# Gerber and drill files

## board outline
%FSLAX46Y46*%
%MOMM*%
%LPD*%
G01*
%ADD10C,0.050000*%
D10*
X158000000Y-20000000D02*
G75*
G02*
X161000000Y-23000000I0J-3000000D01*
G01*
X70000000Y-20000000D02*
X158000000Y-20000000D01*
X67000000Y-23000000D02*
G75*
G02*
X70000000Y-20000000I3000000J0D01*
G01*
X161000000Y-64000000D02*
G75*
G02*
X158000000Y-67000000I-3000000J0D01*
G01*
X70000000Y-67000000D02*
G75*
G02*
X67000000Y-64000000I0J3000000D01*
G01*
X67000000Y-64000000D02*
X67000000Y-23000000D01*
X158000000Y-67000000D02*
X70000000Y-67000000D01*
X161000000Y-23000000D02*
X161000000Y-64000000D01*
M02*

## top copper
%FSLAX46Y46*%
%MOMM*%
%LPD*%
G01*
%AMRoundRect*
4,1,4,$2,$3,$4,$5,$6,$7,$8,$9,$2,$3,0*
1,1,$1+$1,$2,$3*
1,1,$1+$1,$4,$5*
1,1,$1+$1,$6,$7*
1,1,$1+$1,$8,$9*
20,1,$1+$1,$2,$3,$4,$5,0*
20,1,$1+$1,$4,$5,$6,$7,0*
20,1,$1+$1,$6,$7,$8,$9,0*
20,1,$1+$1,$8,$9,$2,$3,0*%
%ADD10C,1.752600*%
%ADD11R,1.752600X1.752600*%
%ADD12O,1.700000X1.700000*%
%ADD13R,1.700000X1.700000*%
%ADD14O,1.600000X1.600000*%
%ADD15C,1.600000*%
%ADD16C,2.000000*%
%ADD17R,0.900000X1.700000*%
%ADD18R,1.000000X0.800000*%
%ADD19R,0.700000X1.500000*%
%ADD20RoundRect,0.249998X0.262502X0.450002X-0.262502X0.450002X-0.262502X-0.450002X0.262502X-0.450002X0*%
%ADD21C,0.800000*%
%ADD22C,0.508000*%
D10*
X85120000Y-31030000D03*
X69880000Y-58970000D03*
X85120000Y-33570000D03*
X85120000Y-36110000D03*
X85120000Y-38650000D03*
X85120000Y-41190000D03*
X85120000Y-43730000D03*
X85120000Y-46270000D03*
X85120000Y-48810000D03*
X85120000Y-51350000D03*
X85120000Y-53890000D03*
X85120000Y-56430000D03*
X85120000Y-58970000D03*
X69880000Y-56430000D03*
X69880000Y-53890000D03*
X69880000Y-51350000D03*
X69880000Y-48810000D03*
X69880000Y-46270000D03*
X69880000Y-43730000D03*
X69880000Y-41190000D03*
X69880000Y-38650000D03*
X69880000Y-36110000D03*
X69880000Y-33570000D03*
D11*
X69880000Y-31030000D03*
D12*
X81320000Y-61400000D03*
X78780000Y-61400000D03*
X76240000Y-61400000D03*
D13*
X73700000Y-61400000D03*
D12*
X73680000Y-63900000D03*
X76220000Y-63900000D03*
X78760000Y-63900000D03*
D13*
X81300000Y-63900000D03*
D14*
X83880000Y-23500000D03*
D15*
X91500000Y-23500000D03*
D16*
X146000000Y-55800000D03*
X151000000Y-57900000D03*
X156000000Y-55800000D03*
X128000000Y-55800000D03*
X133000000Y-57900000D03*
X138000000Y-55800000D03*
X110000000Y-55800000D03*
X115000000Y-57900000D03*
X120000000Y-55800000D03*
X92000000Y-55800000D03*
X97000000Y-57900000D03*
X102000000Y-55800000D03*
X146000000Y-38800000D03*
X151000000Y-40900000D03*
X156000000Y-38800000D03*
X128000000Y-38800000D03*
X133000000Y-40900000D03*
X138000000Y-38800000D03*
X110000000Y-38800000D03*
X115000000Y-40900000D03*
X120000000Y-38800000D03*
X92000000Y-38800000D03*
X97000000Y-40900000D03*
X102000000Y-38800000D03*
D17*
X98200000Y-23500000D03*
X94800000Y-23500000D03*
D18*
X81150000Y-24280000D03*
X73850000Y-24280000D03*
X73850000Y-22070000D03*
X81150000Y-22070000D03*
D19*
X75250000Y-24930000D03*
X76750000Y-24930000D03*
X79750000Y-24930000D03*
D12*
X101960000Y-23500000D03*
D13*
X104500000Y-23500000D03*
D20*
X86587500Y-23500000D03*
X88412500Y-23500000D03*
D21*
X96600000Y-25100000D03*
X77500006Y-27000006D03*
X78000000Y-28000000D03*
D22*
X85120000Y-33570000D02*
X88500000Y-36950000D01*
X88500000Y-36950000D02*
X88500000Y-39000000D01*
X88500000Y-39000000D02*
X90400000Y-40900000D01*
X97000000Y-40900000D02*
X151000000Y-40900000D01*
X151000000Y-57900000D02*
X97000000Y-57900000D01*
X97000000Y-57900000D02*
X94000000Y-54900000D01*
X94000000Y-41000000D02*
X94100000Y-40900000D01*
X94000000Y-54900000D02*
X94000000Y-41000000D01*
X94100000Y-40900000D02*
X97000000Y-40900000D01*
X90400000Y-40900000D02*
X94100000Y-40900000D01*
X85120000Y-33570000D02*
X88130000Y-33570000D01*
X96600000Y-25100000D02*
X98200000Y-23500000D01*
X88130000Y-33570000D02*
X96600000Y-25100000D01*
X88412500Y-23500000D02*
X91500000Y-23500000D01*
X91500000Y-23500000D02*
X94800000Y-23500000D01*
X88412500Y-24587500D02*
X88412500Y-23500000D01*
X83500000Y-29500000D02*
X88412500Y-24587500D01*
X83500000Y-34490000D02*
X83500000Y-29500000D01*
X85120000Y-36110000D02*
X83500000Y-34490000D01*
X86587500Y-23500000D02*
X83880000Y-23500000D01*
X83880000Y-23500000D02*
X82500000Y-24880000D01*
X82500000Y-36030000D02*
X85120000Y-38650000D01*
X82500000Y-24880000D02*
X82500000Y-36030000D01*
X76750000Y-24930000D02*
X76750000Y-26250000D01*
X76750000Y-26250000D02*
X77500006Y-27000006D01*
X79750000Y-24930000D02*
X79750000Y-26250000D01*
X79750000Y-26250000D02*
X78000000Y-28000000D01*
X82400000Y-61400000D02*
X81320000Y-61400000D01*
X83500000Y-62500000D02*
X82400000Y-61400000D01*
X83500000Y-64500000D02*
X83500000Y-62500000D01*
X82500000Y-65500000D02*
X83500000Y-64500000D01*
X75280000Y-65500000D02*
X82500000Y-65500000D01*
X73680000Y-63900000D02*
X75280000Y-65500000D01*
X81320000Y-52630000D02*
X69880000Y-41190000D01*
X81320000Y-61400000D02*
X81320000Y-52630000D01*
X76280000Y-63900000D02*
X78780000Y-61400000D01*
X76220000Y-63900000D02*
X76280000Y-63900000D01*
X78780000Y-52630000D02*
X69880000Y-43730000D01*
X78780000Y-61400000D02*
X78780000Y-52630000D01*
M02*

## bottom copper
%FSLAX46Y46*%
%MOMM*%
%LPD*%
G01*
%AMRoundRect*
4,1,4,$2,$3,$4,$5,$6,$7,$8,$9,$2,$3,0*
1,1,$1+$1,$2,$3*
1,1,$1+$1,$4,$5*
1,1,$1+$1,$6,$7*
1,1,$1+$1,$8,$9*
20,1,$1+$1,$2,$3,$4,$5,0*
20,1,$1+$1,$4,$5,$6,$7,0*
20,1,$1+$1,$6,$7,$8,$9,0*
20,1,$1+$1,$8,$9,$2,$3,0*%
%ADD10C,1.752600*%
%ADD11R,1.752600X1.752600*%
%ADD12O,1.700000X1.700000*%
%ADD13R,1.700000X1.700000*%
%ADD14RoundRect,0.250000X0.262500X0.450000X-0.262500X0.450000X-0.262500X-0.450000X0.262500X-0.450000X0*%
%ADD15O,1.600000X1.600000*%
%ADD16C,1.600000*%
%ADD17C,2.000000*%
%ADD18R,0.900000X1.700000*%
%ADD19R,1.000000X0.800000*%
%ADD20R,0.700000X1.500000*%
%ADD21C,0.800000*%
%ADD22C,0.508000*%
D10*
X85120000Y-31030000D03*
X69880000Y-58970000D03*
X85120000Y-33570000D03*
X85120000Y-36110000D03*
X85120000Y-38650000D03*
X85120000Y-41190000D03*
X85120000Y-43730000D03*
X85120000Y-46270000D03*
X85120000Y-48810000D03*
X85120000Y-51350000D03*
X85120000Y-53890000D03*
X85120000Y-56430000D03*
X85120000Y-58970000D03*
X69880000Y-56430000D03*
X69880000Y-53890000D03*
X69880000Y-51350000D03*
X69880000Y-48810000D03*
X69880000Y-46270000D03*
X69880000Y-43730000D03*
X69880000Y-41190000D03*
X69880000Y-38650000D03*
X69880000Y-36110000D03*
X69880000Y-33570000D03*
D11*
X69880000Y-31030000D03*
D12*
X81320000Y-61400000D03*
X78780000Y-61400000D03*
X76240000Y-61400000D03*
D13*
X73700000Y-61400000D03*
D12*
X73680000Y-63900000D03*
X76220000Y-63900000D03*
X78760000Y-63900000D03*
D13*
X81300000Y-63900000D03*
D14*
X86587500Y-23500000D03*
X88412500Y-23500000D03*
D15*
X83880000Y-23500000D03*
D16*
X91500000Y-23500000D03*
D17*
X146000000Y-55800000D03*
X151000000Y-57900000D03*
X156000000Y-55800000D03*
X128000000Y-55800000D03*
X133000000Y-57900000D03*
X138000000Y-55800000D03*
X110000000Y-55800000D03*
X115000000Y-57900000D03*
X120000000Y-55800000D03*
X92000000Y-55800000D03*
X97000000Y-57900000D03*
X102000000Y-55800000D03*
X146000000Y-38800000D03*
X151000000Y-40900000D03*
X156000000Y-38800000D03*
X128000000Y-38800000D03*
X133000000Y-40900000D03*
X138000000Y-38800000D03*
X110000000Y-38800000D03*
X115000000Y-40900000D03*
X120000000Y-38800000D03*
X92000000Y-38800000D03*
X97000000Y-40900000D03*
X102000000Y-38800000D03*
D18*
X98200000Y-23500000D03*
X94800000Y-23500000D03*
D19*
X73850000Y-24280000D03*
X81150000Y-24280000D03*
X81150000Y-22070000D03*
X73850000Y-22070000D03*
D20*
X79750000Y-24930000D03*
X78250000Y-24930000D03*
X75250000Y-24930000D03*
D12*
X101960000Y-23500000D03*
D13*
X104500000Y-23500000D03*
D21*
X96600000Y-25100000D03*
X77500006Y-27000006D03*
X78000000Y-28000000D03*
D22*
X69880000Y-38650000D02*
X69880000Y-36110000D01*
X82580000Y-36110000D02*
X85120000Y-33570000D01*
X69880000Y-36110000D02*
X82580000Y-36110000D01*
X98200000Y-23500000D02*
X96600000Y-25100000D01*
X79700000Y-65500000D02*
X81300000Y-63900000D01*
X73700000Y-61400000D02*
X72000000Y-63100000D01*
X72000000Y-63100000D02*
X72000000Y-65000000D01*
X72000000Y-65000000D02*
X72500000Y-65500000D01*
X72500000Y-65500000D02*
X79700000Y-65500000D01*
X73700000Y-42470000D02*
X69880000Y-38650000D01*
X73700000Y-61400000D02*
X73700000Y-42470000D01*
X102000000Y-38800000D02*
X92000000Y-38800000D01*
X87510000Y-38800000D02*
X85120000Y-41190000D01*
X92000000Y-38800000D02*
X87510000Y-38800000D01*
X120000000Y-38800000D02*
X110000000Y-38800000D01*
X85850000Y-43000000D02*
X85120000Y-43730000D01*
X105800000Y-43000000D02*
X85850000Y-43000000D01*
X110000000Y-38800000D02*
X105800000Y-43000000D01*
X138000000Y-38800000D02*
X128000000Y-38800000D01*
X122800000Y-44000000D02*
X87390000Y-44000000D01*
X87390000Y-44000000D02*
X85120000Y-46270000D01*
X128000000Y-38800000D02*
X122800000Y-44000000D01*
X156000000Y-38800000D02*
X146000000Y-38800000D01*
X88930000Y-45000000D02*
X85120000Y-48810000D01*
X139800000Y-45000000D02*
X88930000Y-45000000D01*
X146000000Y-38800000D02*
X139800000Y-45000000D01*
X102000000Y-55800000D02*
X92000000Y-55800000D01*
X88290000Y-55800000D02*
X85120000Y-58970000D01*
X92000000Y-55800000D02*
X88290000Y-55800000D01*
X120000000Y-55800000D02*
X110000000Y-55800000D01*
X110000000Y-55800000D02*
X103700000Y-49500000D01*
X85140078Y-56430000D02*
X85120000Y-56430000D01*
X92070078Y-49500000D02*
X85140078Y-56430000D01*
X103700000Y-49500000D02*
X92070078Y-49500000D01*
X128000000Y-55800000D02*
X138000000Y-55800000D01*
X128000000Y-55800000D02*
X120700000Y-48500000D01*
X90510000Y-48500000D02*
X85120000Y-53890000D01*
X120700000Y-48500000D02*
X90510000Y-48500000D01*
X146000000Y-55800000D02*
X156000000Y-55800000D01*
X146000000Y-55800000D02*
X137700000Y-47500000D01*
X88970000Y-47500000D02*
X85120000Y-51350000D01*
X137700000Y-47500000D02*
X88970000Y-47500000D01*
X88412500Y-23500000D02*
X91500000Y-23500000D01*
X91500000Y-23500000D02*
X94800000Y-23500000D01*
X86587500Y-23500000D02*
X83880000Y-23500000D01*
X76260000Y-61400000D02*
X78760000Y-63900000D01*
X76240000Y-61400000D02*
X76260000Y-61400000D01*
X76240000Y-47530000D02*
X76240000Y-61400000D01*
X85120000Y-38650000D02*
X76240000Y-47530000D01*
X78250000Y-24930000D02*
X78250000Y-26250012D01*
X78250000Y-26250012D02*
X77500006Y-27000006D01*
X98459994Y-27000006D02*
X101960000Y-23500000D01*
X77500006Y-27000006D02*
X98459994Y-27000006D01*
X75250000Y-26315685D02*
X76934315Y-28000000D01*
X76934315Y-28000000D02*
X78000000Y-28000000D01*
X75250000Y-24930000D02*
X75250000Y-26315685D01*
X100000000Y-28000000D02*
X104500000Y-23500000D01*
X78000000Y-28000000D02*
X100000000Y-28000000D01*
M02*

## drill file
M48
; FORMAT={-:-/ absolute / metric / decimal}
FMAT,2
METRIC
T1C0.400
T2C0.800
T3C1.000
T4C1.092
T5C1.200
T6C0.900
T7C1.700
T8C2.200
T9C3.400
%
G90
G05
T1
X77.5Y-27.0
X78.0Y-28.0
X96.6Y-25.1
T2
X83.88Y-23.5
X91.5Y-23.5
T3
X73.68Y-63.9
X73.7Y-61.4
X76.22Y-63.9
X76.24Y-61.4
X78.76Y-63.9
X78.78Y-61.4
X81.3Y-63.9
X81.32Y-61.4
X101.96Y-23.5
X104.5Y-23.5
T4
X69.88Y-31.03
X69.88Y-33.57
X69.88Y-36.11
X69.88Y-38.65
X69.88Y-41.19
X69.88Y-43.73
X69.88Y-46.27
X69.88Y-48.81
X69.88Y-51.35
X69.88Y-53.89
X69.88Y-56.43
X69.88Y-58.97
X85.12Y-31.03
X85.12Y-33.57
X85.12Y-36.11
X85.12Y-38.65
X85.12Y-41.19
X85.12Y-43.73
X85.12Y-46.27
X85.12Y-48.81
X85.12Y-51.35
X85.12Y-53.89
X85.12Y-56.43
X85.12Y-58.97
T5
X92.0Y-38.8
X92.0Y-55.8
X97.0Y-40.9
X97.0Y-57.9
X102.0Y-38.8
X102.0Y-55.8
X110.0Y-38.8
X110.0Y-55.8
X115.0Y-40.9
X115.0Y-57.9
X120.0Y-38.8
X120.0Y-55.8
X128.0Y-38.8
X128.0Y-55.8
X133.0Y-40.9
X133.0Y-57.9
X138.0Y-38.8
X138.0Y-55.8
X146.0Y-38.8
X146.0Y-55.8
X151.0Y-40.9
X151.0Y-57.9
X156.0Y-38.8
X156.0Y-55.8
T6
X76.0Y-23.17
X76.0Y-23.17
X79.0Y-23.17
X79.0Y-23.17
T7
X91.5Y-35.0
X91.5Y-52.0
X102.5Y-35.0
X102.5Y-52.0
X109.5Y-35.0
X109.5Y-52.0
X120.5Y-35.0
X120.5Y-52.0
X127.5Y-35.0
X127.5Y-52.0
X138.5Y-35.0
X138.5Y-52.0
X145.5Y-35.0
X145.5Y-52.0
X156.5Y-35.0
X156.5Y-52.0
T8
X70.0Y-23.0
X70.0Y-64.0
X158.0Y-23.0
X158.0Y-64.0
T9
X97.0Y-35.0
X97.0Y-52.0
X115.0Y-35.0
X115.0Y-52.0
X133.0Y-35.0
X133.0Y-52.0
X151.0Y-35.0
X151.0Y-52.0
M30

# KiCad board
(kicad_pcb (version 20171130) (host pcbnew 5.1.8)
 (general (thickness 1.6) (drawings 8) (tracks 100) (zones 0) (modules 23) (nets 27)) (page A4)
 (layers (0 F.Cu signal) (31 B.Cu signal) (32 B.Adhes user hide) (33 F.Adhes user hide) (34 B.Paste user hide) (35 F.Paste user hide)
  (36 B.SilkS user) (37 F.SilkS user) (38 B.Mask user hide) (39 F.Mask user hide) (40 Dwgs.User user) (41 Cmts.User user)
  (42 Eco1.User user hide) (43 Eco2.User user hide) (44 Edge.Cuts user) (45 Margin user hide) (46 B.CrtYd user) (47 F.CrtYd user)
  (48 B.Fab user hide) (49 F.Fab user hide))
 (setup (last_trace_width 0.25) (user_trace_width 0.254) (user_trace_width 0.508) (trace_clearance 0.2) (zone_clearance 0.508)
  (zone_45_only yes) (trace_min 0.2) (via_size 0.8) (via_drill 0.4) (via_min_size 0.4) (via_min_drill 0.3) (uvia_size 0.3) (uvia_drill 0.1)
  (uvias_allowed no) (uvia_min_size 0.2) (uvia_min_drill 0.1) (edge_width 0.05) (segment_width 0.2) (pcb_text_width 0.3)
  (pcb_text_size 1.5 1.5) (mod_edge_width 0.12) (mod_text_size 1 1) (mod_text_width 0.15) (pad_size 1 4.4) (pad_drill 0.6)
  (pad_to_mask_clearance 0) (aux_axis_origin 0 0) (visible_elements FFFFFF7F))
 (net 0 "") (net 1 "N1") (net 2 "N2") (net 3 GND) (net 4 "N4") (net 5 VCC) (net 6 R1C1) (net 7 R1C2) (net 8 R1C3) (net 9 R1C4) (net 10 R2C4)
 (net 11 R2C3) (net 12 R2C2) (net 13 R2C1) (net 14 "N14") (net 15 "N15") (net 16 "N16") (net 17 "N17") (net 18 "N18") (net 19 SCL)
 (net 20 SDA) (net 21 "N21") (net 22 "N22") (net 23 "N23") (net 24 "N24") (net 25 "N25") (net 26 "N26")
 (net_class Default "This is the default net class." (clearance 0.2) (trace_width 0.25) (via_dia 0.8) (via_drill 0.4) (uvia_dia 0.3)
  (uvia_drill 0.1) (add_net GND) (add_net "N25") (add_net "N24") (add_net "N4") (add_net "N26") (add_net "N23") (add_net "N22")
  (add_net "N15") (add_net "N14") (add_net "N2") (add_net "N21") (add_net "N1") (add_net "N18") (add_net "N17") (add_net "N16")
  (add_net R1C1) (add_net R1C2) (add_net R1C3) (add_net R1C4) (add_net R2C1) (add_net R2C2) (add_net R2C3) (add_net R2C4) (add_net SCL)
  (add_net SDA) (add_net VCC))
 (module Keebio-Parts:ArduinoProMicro (layer F.Cu) (at 77.5 45 270)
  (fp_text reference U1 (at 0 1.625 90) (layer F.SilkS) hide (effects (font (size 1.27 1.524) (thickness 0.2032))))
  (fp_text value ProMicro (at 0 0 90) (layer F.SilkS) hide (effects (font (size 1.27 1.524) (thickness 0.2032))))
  (pad 24 thru_hole circle (at -13.97 -7.62 270) (size 1.7526 1.7526) (drill 1.0922) (layers *.Cu *.SilkS *.Mask) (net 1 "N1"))
  (pad 12 thru_hole circle (at 13.97 7.62 270) (size 1.7526 1.7526) (drill 1.0922) (layers *.Cu *.SilkS *.Mask) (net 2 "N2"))
  (pad 23 thru_hole circle (at -11.43 -7.62 270) (size 1.7526 1.7526) (drill 1.0922) (layers *.Cu *.SilkS *.Mask) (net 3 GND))
  (pad 22 thru_hole circle (at -8.89 -7.62 270) (size 1.7526 1.7526) (drill 1.0922) (layers *.Cu *.SilkS *.Mask) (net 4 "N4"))
  (pad 21 thru_hole circle (at -6.35 -7.62 270) (size 1.7526 1.7526) (drill 1.0922) (layers *.Cu *.SilkS *.Mask) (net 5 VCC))
  (pad 20 thru_hole circle (at -3.81 -7.62 270) (size 1.7526 1.7526) (drill 1.0922) (layers *.Cu *.SilkS *.Mask) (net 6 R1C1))
  (pad 19 thru_hole circle (at -1.27 -7.62 270) (size 1.7526 1.7526) (drill 1.0922) (layers *.Cu *.SilkS *.Mask) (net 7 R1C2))
  (pad 18 thru_hole circle (at 1.27 -7.62 270) (size 1.7526 1.7526) (drill 1.0922) (layers *.Cu *.SilkS *.Mask) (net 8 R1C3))
  (pad 17 thru_hole circle (at 3.81 -7.62 270) (size 1.7526 1.7526) (drill 1.0922) (layers *.Cu *.SilkS *.Mask) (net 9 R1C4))
  (pad 16 thru_hole circle (at 6.35 -7.62 270) (size 1.7526 1.7526) (drill 1.0922) (layers *.Cu *.SilkS *.Mask) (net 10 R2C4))
  (pad 15 thru_hole circle (at 8.89 -7.62 270) (size 1.7526 1.7526) (drill 1.0922) (layers *.Cu *.SilkS *.Mask) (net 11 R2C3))
  (pad 14 thru_hole circle (at 11.43 -7.62 270) (size 1.7526 1.7526) (drill 1.0922) (layers *.Cu *.SilkS *.Mask) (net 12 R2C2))
  (pad 13 thru_hole circle (at 13.97 -7.62 270) (size 1.7526 1.7526) (drill 1.0922) (layers *.Cu *.SilkS *.Mask) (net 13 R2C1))
  (pad 11 thru_hole circle (at 11.43 7.62 270) (size 1.7526 1.7526) (drill 1.0922) (layers *.Cu *.SilkS *.Mask) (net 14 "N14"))
  (pad 10 thru_hole circle (at 8.89 7.62 270) (size 1.7526 1.7526) (drill 1.0922) (layers *.Cu *.SilkS *.Mask) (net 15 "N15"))
  (pad 9 thru_hole circle (at 6.35 7.62 270) (size 1.7526 1.7526) (drill 1.0922) (layers *.Cu *.SilkS *.Mask) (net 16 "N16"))
  (pad 8 thru_hole circle (at 3.81 7.62 270) (size 1.7526 1.7526) (drill 1.0922) (layers *.Cu *.SilkS *.Mask) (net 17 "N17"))
  (pad 7 thru_hole circle (at 1.27 7.62 270) (size 1.7526 1.7526) (drill 1.0922) (layers *.Cu *.SilkS *.Mask) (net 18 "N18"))
  (pad 6 thru_hole circle (at -1.27 7.62 270) (size 1.7526 1.7526) (drill 1.0922) (layers *.Cu *.SilkS *.Mask) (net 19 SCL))
  (pad 5 thru_hole circle (at -3.81 7.62 270) (size 1.7526 1.7526) (drill 1.0922) (layers *.Cu *.SilkS *.Mask) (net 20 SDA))
  (pad 4 thru_hole circle (at -6.35 7.62 270) (size 1.7526 1.7526) (drill 1.0922) (layers *.Cu *.SilkS *.Mask) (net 3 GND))
  (pad 3 thru_hole circle (at -8.89 7.62 270) (size 1.7526 1.7526) (drill 1.0922) (layers *.Cu *.SilkS *.Mask) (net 3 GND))
  (pad 2 thru_hole circle (at -11.43 7.62 270) (size 1.7526 1.7526) (drill 1.0922) (layers *.Cu *.SilkS *.Mask) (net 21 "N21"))
  (pad 1 thru_hole rect (at -13.97 7.62 270) (size 1.7526 1.7526) (drill 1.0922) (layers *.Cu *.SilkS *.Mask) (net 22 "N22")))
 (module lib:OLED (layer B.Cu) (at 83.5 63 90)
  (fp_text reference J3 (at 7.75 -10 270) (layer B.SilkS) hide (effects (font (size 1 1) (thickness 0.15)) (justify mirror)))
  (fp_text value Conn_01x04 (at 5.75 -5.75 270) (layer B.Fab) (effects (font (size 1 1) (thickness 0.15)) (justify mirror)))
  (pad 4 thru_hole oval (at 1.6 -2.18 270) (size 1.7 1.7) (drill 1) (layers *.Cu *.Mask) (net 20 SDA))
  (pad 3 thru_hole oval (at 1.6 -4.72 270) (size 1.7 1.7) (drill 1) (layers *.Cu *.Mask) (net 19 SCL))
  (pad 2 thru_hole oval (at 1.6 -7.26 270) (size 1.7 1.7) (drill 1) (layers *.Cu *.Mask) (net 5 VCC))
  (pad 1 thru_hole rect (at 1.6 -9.8 270) (size 1.7 1.7) (drill 1) (layers *.Cu *.Mask) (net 3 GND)))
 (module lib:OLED (layer F.Cu) (at 71.5 65.5 90)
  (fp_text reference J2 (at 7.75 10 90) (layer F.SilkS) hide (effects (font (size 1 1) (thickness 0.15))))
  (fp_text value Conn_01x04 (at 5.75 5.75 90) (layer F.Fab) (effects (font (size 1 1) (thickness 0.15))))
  (pad 4 thru_hole oval (at 1.6 2.18 270) (size 1.7 1.7) (drill 1) (layers *.Cu *.Mask) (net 20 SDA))
  (pad 3 thru_hole oval (at 1.6 4.72 270) (size 1.7 1.7) (drill 1) (layers *.Cu *.Mask) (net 19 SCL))
  (pad 2 thru_hole oval (at 1.6 7.26 270) (size 1.7 1.7) (drill 1) (layers *.Cu *.Mask) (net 5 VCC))
  (pad 1 thru_hole rect (at 1.6 9.8 270) (size 1.7 1.7) (drill 1) (layers *.Cu *.Mask) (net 3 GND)))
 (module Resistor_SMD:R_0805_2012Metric (layer B.Cu) (at 87.5 23.5 180)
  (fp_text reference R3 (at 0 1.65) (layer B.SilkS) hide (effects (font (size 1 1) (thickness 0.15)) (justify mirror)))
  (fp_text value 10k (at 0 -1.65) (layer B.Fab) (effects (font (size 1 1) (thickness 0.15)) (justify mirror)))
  (pad 2 smd roundrect (at 0.9125 0 180) (size 1.025 1.4) (layers B.Cu B.Paste B.Mask) (roundrect_rratio 0.243902) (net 5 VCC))
  (pad 1 smd roundrect (at -0.9125 0 180) (size 1.025 1.4) (layers B.Cu B.Paste B.Mask) (roundrect_rratio 0.243902) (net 4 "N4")))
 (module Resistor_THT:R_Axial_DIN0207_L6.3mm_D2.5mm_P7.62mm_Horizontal (layer F.Cu) (at 91.5 23.5 180)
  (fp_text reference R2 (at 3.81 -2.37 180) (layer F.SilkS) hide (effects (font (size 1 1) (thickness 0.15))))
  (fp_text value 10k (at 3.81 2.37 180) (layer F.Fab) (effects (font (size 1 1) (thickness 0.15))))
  (pad 2 thru_hole oval (at 7.62 0 180) (size 1.6 1.6) (drill 0.8) (layers *.Cu *.Mask) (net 5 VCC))
  (pad 1 thru_hole circle (at 0 0 180) (size 1.6 1.6) (drill 0.8) (layers *.Cu *.Mask) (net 4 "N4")))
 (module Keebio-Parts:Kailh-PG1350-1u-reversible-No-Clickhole (layer F.Cu) (at 151 52)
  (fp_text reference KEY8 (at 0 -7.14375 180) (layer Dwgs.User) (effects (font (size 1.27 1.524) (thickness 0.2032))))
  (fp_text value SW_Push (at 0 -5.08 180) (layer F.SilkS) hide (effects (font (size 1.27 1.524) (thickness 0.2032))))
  (pad "" np_thru_hole circle (at 5.5 0 180) (size 1.7 1.7) (drill 1.7) (layers *.Cu *.Mask))
  (pad "" np_thru_hole circle (at -5.5 0 180) (size 1.7 1.7) (drill 1.7) (layers *.Cu *.Mask))
  (pad 2 thru_hole circle (at -5 3.8 41.9) (size 2 2) (drill 1.2) (layers *.Cu B.Mask) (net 10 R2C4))
  (pad 1 thru_hole circle (at 0 5.9 180) (size 2 2) (drill 1.2) (layers *.Cu *.Mask) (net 3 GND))
  (pad "" np_thru_hole circle (at 0 0 180) (size 3.4 3.4) (drill 3.4) (layers *.Cu *.Mask))
  (pad 2 thru_hole circle (at 5 3.8 41.9) (size 2 2) (drill 1.2) (layers *.Cu F.Mask) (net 10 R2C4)))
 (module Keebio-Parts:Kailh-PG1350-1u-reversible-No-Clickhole (layer F.Cu) (at 133 52)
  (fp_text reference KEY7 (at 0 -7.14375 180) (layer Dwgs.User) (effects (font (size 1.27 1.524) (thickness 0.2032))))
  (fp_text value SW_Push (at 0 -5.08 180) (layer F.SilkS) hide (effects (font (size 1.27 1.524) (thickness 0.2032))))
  (pad "" np_thru_hole circle (at 5.5 0 180) (size 1.7 1.7) (drill 1.7) (layers *.Cu *.Mask))
  (pad "" np_thru_hole circle (at -5.5 0 180) (size 1.7 1.7) (drill 1.7) (layers *.Cu *.Mask))
  (pad 2 thru_hole circle (at -5 3.8 41.9) (size 2 2) (drill 1.2) (layers *.Cu B.Mask) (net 11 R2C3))
  (pad 1 thru_hole circle (at 0 5.9 180) (size 2 2) (drill 1.2) (layers *.Cu *.Mask) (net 3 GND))
  (pad "" np_thru_hole circle (at 0 0 180) (size 3.4 3.4) (drill 3.4) (layers *.Cu *.Mask))
  (pad 2 thru_hole circle (at 5 3.8 41.9) (size 2 2) (drill 1.2) (layers *.Cu F.Mask) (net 11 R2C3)))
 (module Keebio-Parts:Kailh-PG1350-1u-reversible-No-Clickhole (layer F.Cu) (at 115 52)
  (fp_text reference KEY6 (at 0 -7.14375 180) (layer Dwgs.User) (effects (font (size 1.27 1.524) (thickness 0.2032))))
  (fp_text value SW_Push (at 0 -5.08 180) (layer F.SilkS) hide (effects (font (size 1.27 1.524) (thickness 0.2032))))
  (pad "" np_thru_hole circle (at 5.5 0 180) (size 1.7 1.7) (drill 1.7) (layers *.Cu *.Mask))
  (pad "" np_thru_hole circle (at -5.5 0 180) (size 1.7 1.7) (drill 1.7) (layers *.Cu *.Mask))
  (pad 2 thru_hole circle (at -5 3.8 41.9) (size 2 2) (drill 1.2) (layers *.Cu B.Mask) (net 12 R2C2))
  (pad 1 thru_hole circle (at 0 5.9 180) (size 2 2) (drill 1.2) (layers *.Cu *.Mask) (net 3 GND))
  (pad "" np_thru_hole circle (at 0 0 180) (size 3.4 3.4) (drill 3.4) (layers *.Cu *.Mask))
  (pad 2 thru_hole circle (at 5 3.8 41.9) (size 2 2) (drill 1.2) (layers *.Cu F.Mask) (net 12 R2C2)))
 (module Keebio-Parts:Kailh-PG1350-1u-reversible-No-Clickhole (layer F.Cu) (at 97 52)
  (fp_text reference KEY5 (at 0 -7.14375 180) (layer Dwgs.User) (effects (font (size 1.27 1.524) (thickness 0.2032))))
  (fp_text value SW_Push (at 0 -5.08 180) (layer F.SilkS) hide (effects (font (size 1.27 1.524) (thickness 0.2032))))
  (pad "" np_thru_hole circle (at 5.5 0 180) (size 1.7 1.7) (drill 1.7) (layers *.Cu *.Mask))
  (pad "" np_thru_hole circle (at -5.5 0 180) (size 1.7 1.7) (drill 1.7) (layers *.Cu *.Mask))
  (pad 2 thru_hole circle (at -5 3.8 41.9) (size 2 2) (drill 1.2) (layers *.Cu B.Mask) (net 13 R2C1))
  (pad 1 thru_hole circle (at 0 5.9 180) (size 2 2) (drill 1.2) (layers *.Cu *.Mask) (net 3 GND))
  (pad "" np_thru_hole circle (at 0 0 180) (size 3.4 3.4) (drill 3.4) (layers *.Cu *.Mask))
  (pad 2 thru_hole circle (at 5 3.8 41.9) (size 2 2) (drill 1.2) (layers *.Cu F.Mask) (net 13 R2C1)))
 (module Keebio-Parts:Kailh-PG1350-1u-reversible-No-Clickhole (layer F.Cu) (at 151 35)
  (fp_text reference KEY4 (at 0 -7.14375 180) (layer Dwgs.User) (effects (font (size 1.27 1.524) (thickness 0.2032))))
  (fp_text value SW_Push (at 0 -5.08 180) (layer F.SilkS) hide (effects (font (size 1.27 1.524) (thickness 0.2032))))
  (pad "" np_thru_hole circle (at 5.5 0 180) (size 1.7 1.7) (drill 1.7) (layers *.Cu *.Mask))
  (pad "" np_thru_hole circle (at -5.5 0 180) (size 1.7 1.7) (drill 1.7) (layers *.Cu *.Mask))
  (pad 2 thru_hole circle (at -5 3.8 41.9) (size 2 2) (drill 1.2) (layers *.Cu B.Mask) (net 9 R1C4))
  (pad 1 thru_hole circle (at 0 5.9 180) (size 2 2) (drill 1.2) (layers *.Cu *.Mask) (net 3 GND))
  (pad "" np_thru_hole circle (at 0 0 180) (size 3.4 3.4) (drill 3.4) (layers *.Cu *.Mask))
  (pad 2 thru_hole circle (at 5 3.8 41.9) (size 2 2) (drill 1.2) (layers *.Cu F.Mask) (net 9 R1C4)))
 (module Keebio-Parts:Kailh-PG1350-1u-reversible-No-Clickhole (layer F.Cu) (at 133 35)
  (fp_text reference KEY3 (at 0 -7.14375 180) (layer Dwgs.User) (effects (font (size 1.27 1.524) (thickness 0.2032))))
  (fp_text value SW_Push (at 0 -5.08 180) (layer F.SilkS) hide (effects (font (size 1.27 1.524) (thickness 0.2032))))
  (pad "" np_thru_hole circle (at 5.5 0 180) (size 1.7 1.7) (drill 1.7) (layers *.Cu *.Mask))
  (pad "" np_thru_hole circle (at -5.5 0 180) (size 1.7 1.7) (drill 1.7) (layers *.Cu *.Mask))
  (pad 2 thru_hole circle (at -5 3.8 41.9) (size 2 2) (drill 1.2) (layers *.Cu B.Mask) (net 8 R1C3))
  (pad 1 thru_hole circle (at 0 5.9 180) (size 2 2) (drill 1.2) (layers *.Cu *.Mask) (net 3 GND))
  (pad "" np_thru_hole circle (at 0 0 180) (size 3.4 3.4) (drill 3.4) (layers *.Cu *.Mask))
  (pad 2 thru_hole circle (at 5 3.8 41.9) (size 2 2) (drill 1.2) (layers *.Cu F.Mask) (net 8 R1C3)))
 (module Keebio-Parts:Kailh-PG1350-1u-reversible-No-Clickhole (layer F.Cu) (at 115 35)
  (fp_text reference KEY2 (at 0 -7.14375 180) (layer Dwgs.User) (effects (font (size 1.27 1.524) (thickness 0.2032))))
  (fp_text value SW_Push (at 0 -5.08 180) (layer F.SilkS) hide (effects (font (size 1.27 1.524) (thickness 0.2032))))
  (pad "" np_thru_hole circle (at 5.5 0 180) (size 1.7 1.7) (drill 1.7) (layers *.Cu *.Mask))
  (pad "" np_thru_hole circle (at -5.5 0 180) (size 1.7 1.7) (drill 1.7) (layers *.Cu *.Mask))
  (pad 2 thru_hole circle (at -5 3.8 41.9) (size 2 2) (drill 1.2) (layers *.Cu B.Mask) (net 7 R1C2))
  (pad 1 thru_hole circle (at 0 5.9 180) (size 2 2) (drill 1.2) (layers *.Cu *.Mask) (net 3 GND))
  (pad "" np_thru_hole circle (at 0 0 180) (size 3.4 3.4) (drill 3.4) (layers *.Cu *.Mask))
  (pad 2 thru_hole circle (at 5 3.8 41.9) (size 2 2) (drill 1.2) (layers *.Cu F.Mask) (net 7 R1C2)))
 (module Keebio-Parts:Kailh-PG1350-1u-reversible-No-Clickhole (layer F.Cu) (at 97 35)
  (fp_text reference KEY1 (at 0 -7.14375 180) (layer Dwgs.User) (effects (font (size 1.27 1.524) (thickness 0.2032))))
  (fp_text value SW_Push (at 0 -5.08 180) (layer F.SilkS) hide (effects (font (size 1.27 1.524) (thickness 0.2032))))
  (pad "" np_thru_hole circle (at 5.5 0 180) (size 1.7 1.7) (drill 1.7) (layers *.Cu *.Mask))
  (pad "" np_thru_hole circle (at -5.5 0 180) (size 1.7 1.7) (drill 1.7) (layers *.Cu *.Mask))
  (pad 2 thru_hole circle (at -5 3.8 41.9) (size 2 2) (drill 1.2) (layers *.Cu B.Mask) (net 6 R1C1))
  (pad 1 thru_hole circle (at 0 5.9 180) (size 2 2) (drill 1.2) (layers *.Cu *.Mask) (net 3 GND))
  (pad "" np_thru_hole circle (at 0 0 180) (size 3.4 3.4) (drill 3.4) (layers *.Cu *.Mask))
  (pad 2 thru_hole circle (at 5 3.8 41.9) (size 2 2) (drill 1.2) (layers *.Cu F.Mask) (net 6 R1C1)))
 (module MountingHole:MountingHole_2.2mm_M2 (layer F.Cu) (at 70 23)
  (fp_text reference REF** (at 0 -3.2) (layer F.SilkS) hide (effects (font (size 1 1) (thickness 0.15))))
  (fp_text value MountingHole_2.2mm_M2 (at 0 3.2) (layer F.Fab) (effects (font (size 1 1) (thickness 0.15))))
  (pad 1 np_thru_hole circle (at 0 0) (size 2.2 2.2) (drill 2.2) (layers *.Cu *.Mask)))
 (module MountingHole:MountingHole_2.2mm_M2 (layer F.Cu) (at 70 64)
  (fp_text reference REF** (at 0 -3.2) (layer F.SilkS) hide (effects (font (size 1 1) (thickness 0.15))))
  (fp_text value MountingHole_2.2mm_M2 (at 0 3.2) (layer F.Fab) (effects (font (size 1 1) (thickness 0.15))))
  (pad 1 np_thru_hole circle (at 0 0) (size 2.2 2.2) (drill 2.2) (layers *.Cu *.Mask)))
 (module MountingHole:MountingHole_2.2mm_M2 (layer F.Cu) (at 158 64)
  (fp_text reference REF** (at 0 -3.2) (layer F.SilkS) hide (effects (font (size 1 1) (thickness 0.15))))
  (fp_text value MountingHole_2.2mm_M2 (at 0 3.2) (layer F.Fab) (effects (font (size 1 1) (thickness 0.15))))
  (pad 1 np_thru_hole circle (at 0 0) (size 2.2 2.2) (drill 2.2) (layers *.Cu *.Mask)))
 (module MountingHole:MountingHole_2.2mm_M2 (layer F.Cu) (at 158 23)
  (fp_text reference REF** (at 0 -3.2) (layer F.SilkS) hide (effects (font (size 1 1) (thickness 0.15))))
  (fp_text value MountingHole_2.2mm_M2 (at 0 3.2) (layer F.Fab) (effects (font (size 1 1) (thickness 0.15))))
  (pad 1 np_thru_hole circle (at 0 0) (size 2.2 2.2) (drill 2.2) (layers *.Cu *.Mask)))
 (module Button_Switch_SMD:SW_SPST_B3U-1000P (layer F.Cu) (at 96.5 23.5)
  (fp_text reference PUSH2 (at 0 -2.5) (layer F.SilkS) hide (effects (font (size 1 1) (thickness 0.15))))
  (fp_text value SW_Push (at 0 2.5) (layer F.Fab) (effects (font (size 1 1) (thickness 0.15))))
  (pad 2 smd rect (at 1.7 0) (size 0.9 1.7) (layers F.Cu F.Paste F.Mask) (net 3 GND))
  (pad 1 smd rect (at -1.7 0) (size 0.9 1.7) (layers F.Cu F.Paste F.Mask) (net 4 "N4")))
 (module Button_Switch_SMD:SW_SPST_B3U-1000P (layer B.Cu) (at 96.5 23.5)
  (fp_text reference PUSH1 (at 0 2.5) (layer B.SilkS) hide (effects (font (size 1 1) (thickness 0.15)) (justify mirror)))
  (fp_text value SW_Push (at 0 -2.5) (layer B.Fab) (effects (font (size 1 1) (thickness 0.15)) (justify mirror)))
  (pad 2 smd rect (at 1.7 0) (size 0.9 1.7) (layers B.Cu B.Paste B.Mask) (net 3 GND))
  (pad 1 smd rect (at -1.7 0) (size 0.9 1.7) (layers B.Cu B.Paste B.Mask) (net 4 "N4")))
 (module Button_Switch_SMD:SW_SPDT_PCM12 (layer F.Cu) (at 77.5 23.5 180)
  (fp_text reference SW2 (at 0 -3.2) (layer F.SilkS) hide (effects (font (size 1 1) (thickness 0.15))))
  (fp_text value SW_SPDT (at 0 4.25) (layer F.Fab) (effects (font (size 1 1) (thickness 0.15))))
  (pad "" smd rect (at -3.65 -0.78 180) (size 1 0.8) (layers F.Cu F.Paste F.Mask))
  (pad "" smd rect (at 3.65 -0.78 180) (size 1 0.8) (layers F.Cu F.Paste F.Mask))
  (pad "" smd rect (at 3.65 1.43 180) (size 1 0.8) (layers F.Cu F.Paste F.Mask))
  (pad "" smd rect (at -3.65 1.43 180) (size 1 0.8) (layers F.Cu F.Paste F.Mask))
  (pad 3 smd rect (at 2.25 -1.43 180) (size 0.7 1.5) (layers F.Cu F.Paste F.Mask) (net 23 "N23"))
  (pad 2 smd rect (at 0.75 -1.43 180) (size 0.7 1.5) (layers F.Cu F.Paste F.Mask) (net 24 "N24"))
  (pad 1 smd rect (at -2.25 -1.43 180) (size 0.7 1.5) (layers F.Cu F.Paste F.Mask) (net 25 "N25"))
  (pad "" np_thru_hole circle (at 1.5 0.33 180) (size 0.9 0.9) (drill 0.9) (layers *.Cu *.Mask))
  (pad "" np_thru_hole circle (at -1.5 0.33 180) (size 0.9 0.9) (drill 0.9) (layers *.Cu *.Mask)))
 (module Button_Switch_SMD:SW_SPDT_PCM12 (layer B.Cu) (at 77.5 23.5)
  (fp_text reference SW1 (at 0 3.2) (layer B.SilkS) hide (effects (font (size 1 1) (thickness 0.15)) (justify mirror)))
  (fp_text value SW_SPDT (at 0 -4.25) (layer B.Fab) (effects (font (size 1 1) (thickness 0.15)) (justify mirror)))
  (pad "" smd rect (at -3.65 0.78) (size 1 0.8) (layers B.Cu B.Paste B.Mask))
  (pad "" smd rect (at 3.65 0.78) (size 1 0.8) (layers B.Cu B.Paste B.Mask))
  (pad "" smd rect (at 3.65 -1.43) (size 1 0.8) (layers B.Cu B.Paste B.Mask))
  (pad "" smd rect (at -3.65 -1.43) (size 1 0.8) (layers B.Cu B.Paste B.Mask))
  (pad 3 smd rect (at 2.25 1.43) (size 0.7 1.5) (layers B.Cu B.Paste B.Mask) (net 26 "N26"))
  (pad 2 smd rect (at 0.75 1.43) (size 0.7 1.5) (layers B.Cu B.Paste B.Mask) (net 24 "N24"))
  (pad 1 smd rect (at -2.25 1.43) (size 0.7 1.5) (layers B.Cu B.Paste B.Mask) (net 25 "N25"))
  (pad "" np_thru_hole circle (at 1.5 -0.33) (size 0.9 0.9) (drill 0.9) (layers *.Cu *.Mask))
  (pad "" np_thru_hole circle (at -1.5 -0.33) (size 0.9 0.9) (drill 0.9) (layers *.Cu *.Mask)))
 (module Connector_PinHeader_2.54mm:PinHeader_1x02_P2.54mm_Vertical (layer F.Cu) (at 104.5 23.5 270)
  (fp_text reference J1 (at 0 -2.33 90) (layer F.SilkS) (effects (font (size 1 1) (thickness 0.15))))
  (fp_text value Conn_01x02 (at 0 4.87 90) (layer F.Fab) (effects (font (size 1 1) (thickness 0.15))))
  (pad 2 thru_hole oval (at 0 2.54 270) (size 1.7 1.7) (drill 1) (layers *.Cu *.Mask) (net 24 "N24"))
  (pad 1 thru_hole rect (at 0 0 270) (size 1.7 1.7) (drill 1) (layers *.Cu *.Mask) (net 25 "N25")))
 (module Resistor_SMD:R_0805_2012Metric (layer F.Cu) (at 87.5 23.5 180)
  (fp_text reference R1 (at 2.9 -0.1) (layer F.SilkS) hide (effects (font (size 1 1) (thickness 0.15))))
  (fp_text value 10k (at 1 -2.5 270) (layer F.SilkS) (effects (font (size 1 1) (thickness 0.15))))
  (pad 2 smd roundrect (at 0.9125 0 180) (size 1.025 1.4) (layers F.Cu F.Paste F.Mask) (roundrect_rratio 0.2439004878048781) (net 5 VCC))
  (pad 1 smd roundrect (at -0.9125 0 180) (size 1.025 1.4) (layers F.Cu F.Paste F.Mask) (roundrect_rratio 0.2439004878048781) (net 4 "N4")))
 (gr_arc (start 158 23) (end 161 23) (angle -90) (layer Edge.Cuts) (width 0.05))
 (gr_line (start 70 20) (end 158 20) (layer Edge.Cuts) (width 0.05))
 (gr_arc (start 70 23) (end 70 20) (angle -90) (layer Edge.Cuts) (width 0.05))
 (gr_arc (start 158 64) (end 158 67) (angle -90) (layer Edge.Cuts) (width 0.05))
 (gr_arc (start 70 64) (end 67 64) (angle -90) (layer Edge.Cuts) (width 0.05))
 (gr_line (start 67 64) (end 67 23) (layer Edge.Cuts) (width 0.05))
 (gr_line (start 158 67) (end 70 67) (layer Edge.Cuts) (width 0.05))
 (gr_line (start 161 23) (end 161 64) (layer Edge.Cuts) (width 0.05))
 (segment (start 85.12 33.57) (end 88.5 36.95) (width 0.508) (layer F.Cu) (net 3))
 (segment (start 88.5 36.95) (end 88.5 39) (width 0.508) (layer F.Cu) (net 3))
 (segment (start 88.5 39) (end 90.4 40.9) (width 0.508) (layer F.Cu) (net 3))
 (segment (start 97 40.9) (end 151 40.9) (width 0.508) (layer F.Cu) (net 3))
 (segment (start 151 57.9) (end 97 57.9) (width 0.508) (layer F.Cu) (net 3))
 (segment (start 97 57.9) (end 94 54.9) (width 0.508) (layer F.Cu) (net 3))
 (segment (start 94 41) (end 94.1 40.9) (width 0.508) (layer F.Cu) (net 3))
 (segment (start 94 54.9) (end 94 41) (width 0.508) (layer F.Cu) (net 3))
 (segment (start 94.1 40.9) (end 97 40.9) (width 0.508) (layer F.Cu) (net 3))
 (segment (start 90.4 40.9) (end 94.1 40.9) (width 0.508) (layer F.Cu) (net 3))
 (segment (start 69.88 38.65) (end 69.88 36.11) (width 0.508) (layer B.Cu) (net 3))
 (segment (start 82.58 36.11) (end 85.12 33.57) (width 0.508) (layer B.Cu) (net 3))
 (segment (start 69.88 36.11) (end 82.58 36.11) (width 0.508) (layer B.Cu) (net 3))
 (segment (start 85.12 33.57) (end 88.13 33.57) (width 0.508) (layer F.Cu) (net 3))
 (via (at 96.6 25.1) (size 0.8) (drill 0.4) (layers F.Cu B.Cu) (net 3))
 (segment (start 98.2 23.5) (end 96.6 25.1) (width 0.508) (layer B.Cu) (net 3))
 (segment (start 96.6 25.1) (end 98.2 23.5) (width 0.508) (layer F.Cu) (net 3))
 (segment (start 88.13 33.57) (end 96.6 25.1) (width 0.508) (layer F.Cu) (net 3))
 (segment (start 79.7 65.5) (end 81.3 63.9) (width 0.508) (layer B.Cu) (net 3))
 (segment (start 73.7 61.4) (end 72 63.1) (width 0.508) (layer B.Cu) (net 3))
 (segment (start 72 63.1) (end 72 65) (width 0.508) (layer B.Cu) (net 3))
 (segment (start 72 65) (end 72.5 65.5) (width 0.508) (layer B.Cu) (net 3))
 (segment (start 72.5 65.5) (end 79.7 65.5) (width 0.508) (layer B.Cu) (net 3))
 (segment (start 73.7 42.47) (end 69.88 38.65) (width 0.508) (layer B.Cu) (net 3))
 (segment (start 73.7 61.4) (end 73.7 42.47) (width 0.508) (layer B.Cu) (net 3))
 (segment (start 102 38.8) (end 92 38.8) (width 0.508) (layer B.Cu) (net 6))
 (segment (start 87.51 38.8) (end 85.12 41.19) (width 0.508) (layer B.Cu) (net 6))
 (segment (start 92 38.8) (end 87.51 38.8) (width 0.508) (layer B.Cu) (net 6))
 (segment (start 120 38.8) (end 110 38.8) (width 0.508) (layer B.Cu) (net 7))
 (segment (start 85.85 43) (end 85.12 43.73) (width 0.508) (layer B.Cu) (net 7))
 (segment (start 105.8 43) (end 85.85 43) (width 0.508) (layer B.Cu) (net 7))
 (segment (start 110 38.8) (end 105.8 43) (width 0.508) (layer B.Cu) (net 7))
 (segment (start 138 38.8) (end 128 38.8) (width 0.508) (layer B.Cu) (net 8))
 (segment (start 122.8 44) (end 87.39 44) (width 0.508) (layer B.Cu) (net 8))
 (segment (start 87.39 44) (end 85.12 46.27) (width 0.508) (layer B.Cu) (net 8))
 (segment (start 128 38.8) (end 122.8 44) (width 0.508) (layer B.Cu) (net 8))
 (segment (start 156 38.8) (end 146 38.8) (width 0.508) (layer B.Cu) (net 9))
 (segment (start 88.93 45) (end 85.12 48.81) (width 0.508) (layer B.Cu) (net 9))
 (segment (start 139.8 45) (end 88.93 45) (width 0.508) (layer B.Cu) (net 9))
 (segment (start 146 38.8) (end 139.8 45) (width 0.508) (layer B.Cu) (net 9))
 (segment (start 102 55.8) (end 92 55.8) (width 0.508) (layer B.Cu) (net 13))
 (segment (start 88.29 55.8) (end 85.12 58.97) (width 0.508) (layer B.Cu) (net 13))
 (segment (start 92 55.8) (end 88.29 55.8) (width 0.508) (layer B.Cu) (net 13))
 (segment (start 120 55.8) (end 110 55.8) (width 0.508) (layer B.Cu) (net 12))
 (segment (start 110 55.8) (end 103.7 49.5) (width 0.508) (layer B.Cu) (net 12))
 (segment (start 85.140078 56.43) (end 85.12 56.43) (width 0.508) (layer B.Cu) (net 12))
 (segment (start 92.070078 49.5) (end 85.140078 56.43) (width 0.508) (layer B.Cu) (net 12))
 (segment (start 103.7 49.5) (end 92.070078 49.5) (width 0.508) (layer B.Cu) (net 12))
 (segment (start 128 55.8) (end 138 55.8) (width 0.508) (layer B.Cu) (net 11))
 (segment (start 128 55.8) (end 120.7 48.5) (width 0.508) (layer B.Cu) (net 11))
 (segment (start 90.51 48.5) (end 85.12 53.89) (width 0.508) (layer B.Cu) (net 11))
 (segment (start 120.7 48.5) (end 90.51 48.5) (width 0.508) (layer B.Cu) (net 11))
 (segment (start 146 55.8) (end 156 55.8) (width 0.508) (layer B.Cu) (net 10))
 (segment (start 146 55.8) (end 137.7 47.5) (width 0.508) (layer B.Cu) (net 10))
 (segment (start 88.97 47.5) (end 85.12 51.35) (width 0.508) (layer B.Cu) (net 10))
 (segment (start 137.7 47.5) (end 88.97 47.5) (width 0.508) (layer B.Cu) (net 10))
 (segment (start 88.4125 23.5) (end 91.5 23.5) (width 0.508) (layer F.Cu) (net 4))
 (segment (start 88.4125 23.5) (end 91.5 23.5) (width 0.508) (layer B.Cu) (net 4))
 (segment (start 91.5 23.5) (end 94.8 23.5) (width 0.508) (layer B.Cu) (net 4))
 (segment (start 91.5 23.5) (end 94.8 23.5) (width 0.508) (layer F.Cu) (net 4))
 (segment (start 88.4125 24.5875) (end 88.4125 23.5) (width 0.508) (layer F.Cu) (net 4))
 (segment (start 83.5 29.5) (end 88.4125 24.5875) (width 0.508) (layer F.Cu) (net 4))
 (segment (start 83.5 34.49) (end 83.5 29.5) (width 0.508) (layer F.Cu) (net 4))
 (segment (start 85.12 36.11) (end 83.5 34.49) (width 0.508) (layer F.Cu) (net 4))
 (segment (start 86.5875 23.5) (end 83.88 23.5) (width 0.508) (layer F.Cu) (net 5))
 (segment (start 86.5875 23.5) (end 83.88 23.5) (width 0.508) (layer B.Cu) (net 5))
 (segment (start 83.88 23.5) (end 82.5 24.88) (width 0.508) (layer F.Cu) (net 5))
 (segment (start 82.5 36.03) (end 85.12 38.65) (width 0.508) (layer F.Cu) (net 5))
 (segment (start 82.5 24.88) (end 82.5 36.03) (width 0.508) (layer F.Cu) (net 5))
 (segment (start 76.26 61.4) (end 78.76 63.9) (width 0.508) (layer B.Cu) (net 5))
 (segment (start 76.24 61.4) (end 76.26 61.4) (width 0.508) (layer B.Cu) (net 5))
 (segment (start 76.24 47.53) (end 76.24 61.4) (width 0.508) (layer B.Cu) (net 5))
 (segment (start 85.12 38.65) (end 76.24 47.53) (width 0.508) (layer B.Cu) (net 5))
 (via (at 77.500006 27.000006) (size 0.8) (drill 0.4) (layers F.Cu B.Cu) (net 24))
 (segment (start 76.75 24.93) (end 76.75 26.25) (width 0.508) (layer F.Cu) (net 24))
 (segment (start 76.75 26.25) (end 77.500006 27.000006) (width 0.508) (layer F.Cu) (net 24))
 (segment (start 78.25 24.93) (end 78.25 26.250012) (width 0.508) (layer B.Cu) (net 24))
 (segment (start 78.25 26.250012) (end 77.500006 27.000006) (width 0.508) (layer B.Cu) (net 24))
 (segment (start 98.459994 27.000006) (end 101.96 23.5) (width 0.508) (layer B.Cu) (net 24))
 (segment (start 77.500006 27.000006) (end 98.459994 27.000006) (width 0.508) (layer B.Cu) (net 24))
 (via (at 78 28) (size 0.8) (drill 0.4) (layers F.Cu B.Cu) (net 25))
 (segment (start 79.75 24.93) (end 79.75 26.25) (width 0.508) (layer F.Cu) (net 25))
 (segment (start 75.25 26.315685) (end 76.934315 28) (width 0.508) (layer B.Cu) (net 25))
 (segment (start 79.75 26.25) (end 78 28) (width 0.508) (layer F.Cu) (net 25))
 (segment (start 76.934315 28) (end 78 28) (width 0.508) (layer B.Cu) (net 25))
 (segment (start 75.25 24.93) (end 75.25 26.315685) (width 0.508) (layer B.Cu) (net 25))
 (segment (start 100 28) (end 104.5 23.5) (width 0.508) (layer B.Cu) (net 25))
 (segment (start 78 28) (end 100 28) (width 0.508) (layer B.Cu) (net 25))
 (segment (start 82.4 61.4) (end 81.32 61.4) (width 0.508) (layer F.Cu) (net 20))
 (segment (start 83.5 62.5) (end 82.4 61.4) (width 0.508) (layer F.Cu) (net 20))
 (segment (start 83.5 64.5) (end 83.5 62.5) (width 0.508) (layer F.Cu) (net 20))
 (segment (start 82.5 65.5) (end 83.5 64.5) (width 0.508) (layer F.Cu) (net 20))
 (segment (start 75.28 65.5) (end 82.5 65.5) (width 0.508) (layer F.Cu) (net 20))
 (segment (start 73.68 63.9) (end 75.28 65.5) (width 0.508) (layer F.Cu) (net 20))
 (segment (start 81.32 52.63) (end 69.88 41.19) (width 0.508) (layer F.Cu) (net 20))
 (segment (start 81.32 61.4) (end 81.32 52.63) (width 0.508) (layer F.Cu) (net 20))
 (segment (start 76.28 63.9) (end 78.78 61.4) (width 0.508) (layer F.Cu) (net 19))
 (segment (start 76.22 63.9) (end 76.28 63.9) (width 0.508) (layer F.Cu) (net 19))
 (segment (start 78.78 52.63) (end 69.88 43.73) (width 0.508) (layer F.Cu) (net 19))
 (segment (start 78.78 61.4) (end 78.78 52.63) (width 0.508) (layer F.Cu) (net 19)))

